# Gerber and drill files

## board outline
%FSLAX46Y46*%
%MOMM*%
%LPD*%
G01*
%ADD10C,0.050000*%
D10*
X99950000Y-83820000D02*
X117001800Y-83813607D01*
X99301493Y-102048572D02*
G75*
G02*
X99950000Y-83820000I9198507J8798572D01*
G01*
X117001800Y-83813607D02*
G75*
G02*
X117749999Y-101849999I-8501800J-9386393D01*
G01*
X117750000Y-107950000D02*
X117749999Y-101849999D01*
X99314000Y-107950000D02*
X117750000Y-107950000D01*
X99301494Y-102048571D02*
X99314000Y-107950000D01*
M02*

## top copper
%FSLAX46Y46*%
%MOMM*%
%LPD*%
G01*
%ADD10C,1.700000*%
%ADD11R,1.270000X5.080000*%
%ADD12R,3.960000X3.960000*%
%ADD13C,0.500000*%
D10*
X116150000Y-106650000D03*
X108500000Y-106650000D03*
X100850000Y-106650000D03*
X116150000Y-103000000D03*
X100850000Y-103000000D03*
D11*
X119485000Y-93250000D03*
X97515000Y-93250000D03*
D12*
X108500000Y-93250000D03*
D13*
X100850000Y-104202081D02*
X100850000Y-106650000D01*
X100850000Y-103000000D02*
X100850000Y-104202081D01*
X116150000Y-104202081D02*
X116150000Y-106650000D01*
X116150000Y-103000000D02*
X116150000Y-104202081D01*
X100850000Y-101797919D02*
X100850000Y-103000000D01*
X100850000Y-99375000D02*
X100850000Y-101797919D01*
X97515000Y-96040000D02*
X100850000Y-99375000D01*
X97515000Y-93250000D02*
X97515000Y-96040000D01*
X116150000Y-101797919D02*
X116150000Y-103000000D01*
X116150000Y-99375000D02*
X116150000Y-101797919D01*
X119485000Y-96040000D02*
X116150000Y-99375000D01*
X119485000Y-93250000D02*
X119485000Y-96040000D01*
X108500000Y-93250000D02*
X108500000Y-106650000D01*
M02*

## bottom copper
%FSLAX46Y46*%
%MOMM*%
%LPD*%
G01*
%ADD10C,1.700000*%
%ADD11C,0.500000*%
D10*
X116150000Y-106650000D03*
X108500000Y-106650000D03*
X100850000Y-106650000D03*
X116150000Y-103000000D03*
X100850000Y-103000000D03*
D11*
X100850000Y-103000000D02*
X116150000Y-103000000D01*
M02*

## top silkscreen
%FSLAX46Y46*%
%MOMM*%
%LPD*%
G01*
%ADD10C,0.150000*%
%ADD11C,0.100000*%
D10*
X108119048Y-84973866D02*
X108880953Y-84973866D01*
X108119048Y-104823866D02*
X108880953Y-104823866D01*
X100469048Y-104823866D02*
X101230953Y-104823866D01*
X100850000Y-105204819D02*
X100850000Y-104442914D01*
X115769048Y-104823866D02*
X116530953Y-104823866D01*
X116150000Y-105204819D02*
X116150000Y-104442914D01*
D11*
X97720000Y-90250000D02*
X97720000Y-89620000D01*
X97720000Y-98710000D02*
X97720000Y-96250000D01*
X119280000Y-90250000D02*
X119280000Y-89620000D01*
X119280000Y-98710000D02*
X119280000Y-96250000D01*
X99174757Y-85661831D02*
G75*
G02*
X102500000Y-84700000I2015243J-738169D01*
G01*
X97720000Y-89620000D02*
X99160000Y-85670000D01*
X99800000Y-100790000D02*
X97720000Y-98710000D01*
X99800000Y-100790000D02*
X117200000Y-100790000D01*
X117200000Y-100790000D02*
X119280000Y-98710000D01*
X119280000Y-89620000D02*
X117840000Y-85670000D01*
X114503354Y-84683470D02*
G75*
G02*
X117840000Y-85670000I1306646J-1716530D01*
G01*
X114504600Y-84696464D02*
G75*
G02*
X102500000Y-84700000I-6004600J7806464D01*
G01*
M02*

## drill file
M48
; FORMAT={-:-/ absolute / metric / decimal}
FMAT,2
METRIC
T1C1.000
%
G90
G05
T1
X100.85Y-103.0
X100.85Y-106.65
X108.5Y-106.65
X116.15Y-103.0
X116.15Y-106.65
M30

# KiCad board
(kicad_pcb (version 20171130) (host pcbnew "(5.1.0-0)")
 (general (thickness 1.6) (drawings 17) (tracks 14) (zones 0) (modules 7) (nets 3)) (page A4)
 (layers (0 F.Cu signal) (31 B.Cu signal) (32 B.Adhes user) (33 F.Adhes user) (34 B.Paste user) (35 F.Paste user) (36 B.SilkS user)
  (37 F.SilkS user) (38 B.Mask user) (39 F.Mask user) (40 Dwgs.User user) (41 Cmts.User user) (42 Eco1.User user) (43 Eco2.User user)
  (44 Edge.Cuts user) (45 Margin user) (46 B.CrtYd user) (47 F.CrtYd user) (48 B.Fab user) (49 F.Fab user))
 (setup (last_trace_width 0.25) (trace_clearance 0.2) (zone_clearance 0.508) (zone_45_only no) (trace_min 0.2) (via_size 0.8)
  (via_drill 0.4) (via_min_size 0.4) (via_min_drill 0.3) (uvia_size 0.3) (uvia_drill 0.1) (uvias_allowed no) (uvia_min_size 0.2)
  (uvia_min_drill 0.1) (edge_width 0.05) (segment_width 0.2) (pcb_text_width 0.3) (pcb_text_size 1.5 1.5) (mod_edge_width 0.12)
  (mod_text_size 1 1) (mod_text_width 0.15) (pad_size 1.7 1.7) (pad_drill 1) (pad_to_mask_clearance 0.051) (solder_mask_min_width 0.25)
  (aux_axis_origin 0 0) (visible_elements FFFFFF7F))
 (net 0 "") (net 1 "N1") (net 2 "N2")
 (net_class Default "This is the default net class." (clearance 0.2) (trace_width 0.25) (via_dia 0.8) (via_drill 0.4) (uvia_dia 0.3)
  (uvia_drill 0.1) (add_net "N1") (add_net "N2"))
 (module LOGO (layer B.Cu) (at 108.5 98.65 180)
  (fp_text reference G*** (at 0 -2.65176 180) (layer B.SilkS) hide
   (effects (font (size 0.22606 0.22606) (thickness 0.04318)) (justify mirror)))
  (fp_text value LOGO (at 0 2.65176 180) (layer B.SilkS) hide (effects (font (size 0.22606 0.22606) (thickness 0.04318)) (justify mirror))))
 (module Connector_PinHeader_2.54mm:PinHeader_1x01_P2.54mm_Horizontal (layer B.Cu) (at 116.15 106.65 270)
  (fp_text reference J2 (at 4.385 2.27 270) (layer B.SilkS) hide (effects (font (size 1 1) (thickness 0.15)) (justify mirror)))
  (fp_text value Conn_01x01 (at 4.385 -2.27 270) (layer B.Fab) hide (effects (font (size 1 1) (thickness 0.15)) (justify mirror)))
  (pad 1 thru_hole circle (at 0 0 270) (size 1.7 1.7) (drill 1) (layers *.Cu *.Mask) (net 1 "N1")))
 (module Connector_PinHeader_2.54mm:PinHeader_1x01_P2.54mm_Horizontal (layer F.Cu) (at 108.5 106.65 270)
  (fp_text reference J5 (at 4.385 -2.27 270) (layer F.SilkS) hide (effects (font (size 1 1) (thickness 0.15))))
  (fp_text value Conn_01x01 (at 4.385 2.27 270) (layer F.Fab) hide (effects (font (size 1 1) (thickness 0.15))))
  (pad 1 thru_hole circle (at 0 0 270) (size 1.7 1.7) (drill 1) (layers *.Cu *.Mask) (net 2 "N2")))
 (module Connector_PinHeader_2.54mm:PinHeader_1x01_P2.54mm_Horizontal (layer B.Cu) (at 100.85 106.65 270)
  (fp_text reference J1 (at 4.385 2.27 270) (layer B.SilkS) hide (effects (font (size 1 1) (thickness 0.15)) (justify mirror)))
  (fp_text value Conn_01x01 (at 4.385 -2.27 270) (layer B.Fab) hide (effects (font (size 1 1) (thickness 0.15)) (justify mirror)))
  (pad 1 thru_hole circle (at 0 0 270) (size 1.7 1.7) (drill 1) (layers *.Cu *.Mask) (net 1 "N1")))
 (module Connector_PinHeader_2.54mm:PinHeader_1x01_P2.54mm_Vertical (layer B.Cu) (at 116.15 103)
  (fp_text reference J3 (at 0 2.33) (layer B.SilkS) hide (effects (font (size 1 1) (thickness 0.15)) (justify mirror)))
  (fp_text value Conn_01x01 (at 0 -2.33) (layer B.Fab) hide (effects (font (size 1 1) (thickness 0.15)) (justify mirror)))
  (pad 1 thru_hole circle (at 0 0) (size 1.7 1.7) (drill 1) (layers *.Cu *.Mask) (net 1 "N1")))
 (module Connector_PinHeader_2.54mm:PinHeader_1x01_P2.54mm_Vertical (layer B.Cu) (at 100.85 103)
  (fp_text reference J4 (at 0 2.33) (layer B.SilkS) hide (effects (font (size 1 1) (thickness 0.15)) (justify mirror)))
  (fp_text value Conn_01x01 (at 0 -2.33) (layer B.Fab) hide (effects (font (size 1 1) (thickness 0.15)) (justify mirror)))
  (pad 1 thru_hole circle (at 0 0) (size 1.7 1.7) (drill 1) (layers *.Cu *.Mask) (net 1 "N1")))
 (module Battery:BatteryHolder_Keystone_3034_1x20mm (layer F.Cu) (at 108.5 93.25 180)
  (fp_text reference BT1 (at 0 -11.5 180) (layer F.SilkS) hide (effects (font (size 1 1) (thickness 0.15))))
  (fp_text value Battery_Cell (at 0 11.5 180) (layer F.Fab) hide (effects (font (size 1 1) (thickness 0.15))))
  (fp_line (start 10.78 3) (end 10.78 3.63) (layer F.SilkS) (width 0.1))
  (fp_line (start 10.78 -5.46) (end 10.78 -3) (layer F.SilkS) (width 0.1))
  (fp_line (start -10.78 3) (end -10.78 3.63) (layer F.SilkS) (width 0.1))
  (fp_line (start -10.78 -5.46) (end -10.78 -3) (layer F.SilkS) (width 0.1))
  (fp_arc (start 7.31 6.85) (end 6 8.55) (angle -107.5) (layer F.SilkS) (width 0.1))
  (fp_line (start 10.78 3.63) (end 9.34 7.58) (layer F.SilkS) (width 0.1))
  (fp_line (start 8.7 -7.54) (end 10.78 -5.46) (layer F.SilkS) (width 0.1))
  (fp_line (start 8.7 -7.54) (end -8.7 -7.54) (layer F.SilkS) (width 0.1))
  (fp_line (start -8.7 -7.54) (end -10.78 -5.46) (layer F.SilkS) (width 0.1))
  (fp_line (start -10.78 3.63) (end -9.34 7.58) (layer F.SilkS) (width 0.1))
  (fp_arc (start -7.31 6.85) (end -9.34 7.58) (angle -107.5) (layer F.SilkS) (width 0.1))
  (fp_arc (start 0 16.36) (end 6 8.55) (angle -75.1) (layer F.SilkS) (width 0.1))
  (pad 1 smd rect (at -10.985 0 180) (size 1.27 5.08) (layers F.Cu F.Paste F.Mask) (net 1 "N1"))
  (pad 1 smd rect (at 10.985 0 180) (size 1.27 5.08) (layers F.Cu F.Paste F.Mask) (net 1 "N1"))
  (pad 2 smd rect (at 0 0 180) (size 3.96 3.96) (layers F.Cu F.Paste F.Mask) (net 2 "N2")))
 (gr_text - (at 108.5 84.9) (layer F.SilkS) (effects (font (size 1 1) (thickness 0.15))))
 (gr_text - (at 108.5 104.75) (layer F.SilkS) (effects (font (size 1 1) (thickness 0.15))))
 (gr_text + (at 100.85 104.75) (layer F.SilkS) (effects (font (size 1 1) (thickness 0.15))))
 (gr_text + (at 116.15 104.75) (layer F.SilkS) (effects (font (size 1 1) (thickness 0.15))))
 (gr_line (start 99.95 83.82) (end 117.0018 83.813607) (layer Edge.Cuts) (width 0.05))
 (gr_arc (start 108.5 93.25) (end 99.95 83.82) (angle -91.52897716) (layer Edge.Cuts) (width 0.05))
 (gr_arc (start 108.5 93.2) (end 117.749999 101.849999) (angle -90.91123063) (layer Edge.Cuts) (width 0.05))
 (gr_line (start 117.75 107.95) (end 117.749999 101.849999) (layer Edge.Cuts) (width 0.05))
 (gr_line (start 99.314 107.95) (end 117.75 107.95) (layer Edge.Cuts) (width 0.05))
 (gr_line (start 99.301494 102.048571) (end 99.314 107.95) (layer Edge.Cuts) (width 0.05))
 (segment (start 100.85 104.202081) (end 100.85 106.65) (width 0.5) (layer F.Cu) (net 1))
 (segment (start 100.85 103) (end 100.85 104.202081) (width 0.5) (layer F.Cu) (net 1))
 (segment (start 116.15 104.202081) (end 116.15 106.65) (width 0.5) (layer F.Cu) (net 1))
 (segment (start 116.15 103) (end 116.15 104.202081) (width 0.5) (layer F.Cu) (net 1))
 (segment (start 100.85 101.797919) (end 100.85 103) (width 0.5) (layer F.Cu) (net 1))
 (segment (start 100.85 99.375) (end 100.85 101.797919) (width 0.5) (layer F.Cu) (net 1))
 (segment (start 97.515 96.04) (end 100.85 99.375) (width 0.5) (layer F.Cu) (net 1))
 (segment (start 97.515 93.25) (end 97.515 96.04) (width 0.5) (layer F.Cu) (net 1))
 (segment (start 116.15 101.797919) (end 116.15 103) (width 0.5) (layer F.Cu) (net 1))
 (segment (start 116.15 99.375) (end 116.15 101.797919) (width 0.5) (layer F.Cu) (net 1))
 (segment (start 119.485 96.04) (end 116.15 99.375) (width 0.5) (layer F.Cu) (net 1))
 (segment (start 119.485 93.25) (end 119.485 96.04) (width 0.5) (layer F.Cu) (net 1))
 (segment (start 100.85 103) (end 116.15 103) (width 0.5) (layer B.Cu) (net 1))
 (segment (start 108.5 93.25) (end 108.5 106.65) (width 0.5) (layer F.Cu) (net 2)))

